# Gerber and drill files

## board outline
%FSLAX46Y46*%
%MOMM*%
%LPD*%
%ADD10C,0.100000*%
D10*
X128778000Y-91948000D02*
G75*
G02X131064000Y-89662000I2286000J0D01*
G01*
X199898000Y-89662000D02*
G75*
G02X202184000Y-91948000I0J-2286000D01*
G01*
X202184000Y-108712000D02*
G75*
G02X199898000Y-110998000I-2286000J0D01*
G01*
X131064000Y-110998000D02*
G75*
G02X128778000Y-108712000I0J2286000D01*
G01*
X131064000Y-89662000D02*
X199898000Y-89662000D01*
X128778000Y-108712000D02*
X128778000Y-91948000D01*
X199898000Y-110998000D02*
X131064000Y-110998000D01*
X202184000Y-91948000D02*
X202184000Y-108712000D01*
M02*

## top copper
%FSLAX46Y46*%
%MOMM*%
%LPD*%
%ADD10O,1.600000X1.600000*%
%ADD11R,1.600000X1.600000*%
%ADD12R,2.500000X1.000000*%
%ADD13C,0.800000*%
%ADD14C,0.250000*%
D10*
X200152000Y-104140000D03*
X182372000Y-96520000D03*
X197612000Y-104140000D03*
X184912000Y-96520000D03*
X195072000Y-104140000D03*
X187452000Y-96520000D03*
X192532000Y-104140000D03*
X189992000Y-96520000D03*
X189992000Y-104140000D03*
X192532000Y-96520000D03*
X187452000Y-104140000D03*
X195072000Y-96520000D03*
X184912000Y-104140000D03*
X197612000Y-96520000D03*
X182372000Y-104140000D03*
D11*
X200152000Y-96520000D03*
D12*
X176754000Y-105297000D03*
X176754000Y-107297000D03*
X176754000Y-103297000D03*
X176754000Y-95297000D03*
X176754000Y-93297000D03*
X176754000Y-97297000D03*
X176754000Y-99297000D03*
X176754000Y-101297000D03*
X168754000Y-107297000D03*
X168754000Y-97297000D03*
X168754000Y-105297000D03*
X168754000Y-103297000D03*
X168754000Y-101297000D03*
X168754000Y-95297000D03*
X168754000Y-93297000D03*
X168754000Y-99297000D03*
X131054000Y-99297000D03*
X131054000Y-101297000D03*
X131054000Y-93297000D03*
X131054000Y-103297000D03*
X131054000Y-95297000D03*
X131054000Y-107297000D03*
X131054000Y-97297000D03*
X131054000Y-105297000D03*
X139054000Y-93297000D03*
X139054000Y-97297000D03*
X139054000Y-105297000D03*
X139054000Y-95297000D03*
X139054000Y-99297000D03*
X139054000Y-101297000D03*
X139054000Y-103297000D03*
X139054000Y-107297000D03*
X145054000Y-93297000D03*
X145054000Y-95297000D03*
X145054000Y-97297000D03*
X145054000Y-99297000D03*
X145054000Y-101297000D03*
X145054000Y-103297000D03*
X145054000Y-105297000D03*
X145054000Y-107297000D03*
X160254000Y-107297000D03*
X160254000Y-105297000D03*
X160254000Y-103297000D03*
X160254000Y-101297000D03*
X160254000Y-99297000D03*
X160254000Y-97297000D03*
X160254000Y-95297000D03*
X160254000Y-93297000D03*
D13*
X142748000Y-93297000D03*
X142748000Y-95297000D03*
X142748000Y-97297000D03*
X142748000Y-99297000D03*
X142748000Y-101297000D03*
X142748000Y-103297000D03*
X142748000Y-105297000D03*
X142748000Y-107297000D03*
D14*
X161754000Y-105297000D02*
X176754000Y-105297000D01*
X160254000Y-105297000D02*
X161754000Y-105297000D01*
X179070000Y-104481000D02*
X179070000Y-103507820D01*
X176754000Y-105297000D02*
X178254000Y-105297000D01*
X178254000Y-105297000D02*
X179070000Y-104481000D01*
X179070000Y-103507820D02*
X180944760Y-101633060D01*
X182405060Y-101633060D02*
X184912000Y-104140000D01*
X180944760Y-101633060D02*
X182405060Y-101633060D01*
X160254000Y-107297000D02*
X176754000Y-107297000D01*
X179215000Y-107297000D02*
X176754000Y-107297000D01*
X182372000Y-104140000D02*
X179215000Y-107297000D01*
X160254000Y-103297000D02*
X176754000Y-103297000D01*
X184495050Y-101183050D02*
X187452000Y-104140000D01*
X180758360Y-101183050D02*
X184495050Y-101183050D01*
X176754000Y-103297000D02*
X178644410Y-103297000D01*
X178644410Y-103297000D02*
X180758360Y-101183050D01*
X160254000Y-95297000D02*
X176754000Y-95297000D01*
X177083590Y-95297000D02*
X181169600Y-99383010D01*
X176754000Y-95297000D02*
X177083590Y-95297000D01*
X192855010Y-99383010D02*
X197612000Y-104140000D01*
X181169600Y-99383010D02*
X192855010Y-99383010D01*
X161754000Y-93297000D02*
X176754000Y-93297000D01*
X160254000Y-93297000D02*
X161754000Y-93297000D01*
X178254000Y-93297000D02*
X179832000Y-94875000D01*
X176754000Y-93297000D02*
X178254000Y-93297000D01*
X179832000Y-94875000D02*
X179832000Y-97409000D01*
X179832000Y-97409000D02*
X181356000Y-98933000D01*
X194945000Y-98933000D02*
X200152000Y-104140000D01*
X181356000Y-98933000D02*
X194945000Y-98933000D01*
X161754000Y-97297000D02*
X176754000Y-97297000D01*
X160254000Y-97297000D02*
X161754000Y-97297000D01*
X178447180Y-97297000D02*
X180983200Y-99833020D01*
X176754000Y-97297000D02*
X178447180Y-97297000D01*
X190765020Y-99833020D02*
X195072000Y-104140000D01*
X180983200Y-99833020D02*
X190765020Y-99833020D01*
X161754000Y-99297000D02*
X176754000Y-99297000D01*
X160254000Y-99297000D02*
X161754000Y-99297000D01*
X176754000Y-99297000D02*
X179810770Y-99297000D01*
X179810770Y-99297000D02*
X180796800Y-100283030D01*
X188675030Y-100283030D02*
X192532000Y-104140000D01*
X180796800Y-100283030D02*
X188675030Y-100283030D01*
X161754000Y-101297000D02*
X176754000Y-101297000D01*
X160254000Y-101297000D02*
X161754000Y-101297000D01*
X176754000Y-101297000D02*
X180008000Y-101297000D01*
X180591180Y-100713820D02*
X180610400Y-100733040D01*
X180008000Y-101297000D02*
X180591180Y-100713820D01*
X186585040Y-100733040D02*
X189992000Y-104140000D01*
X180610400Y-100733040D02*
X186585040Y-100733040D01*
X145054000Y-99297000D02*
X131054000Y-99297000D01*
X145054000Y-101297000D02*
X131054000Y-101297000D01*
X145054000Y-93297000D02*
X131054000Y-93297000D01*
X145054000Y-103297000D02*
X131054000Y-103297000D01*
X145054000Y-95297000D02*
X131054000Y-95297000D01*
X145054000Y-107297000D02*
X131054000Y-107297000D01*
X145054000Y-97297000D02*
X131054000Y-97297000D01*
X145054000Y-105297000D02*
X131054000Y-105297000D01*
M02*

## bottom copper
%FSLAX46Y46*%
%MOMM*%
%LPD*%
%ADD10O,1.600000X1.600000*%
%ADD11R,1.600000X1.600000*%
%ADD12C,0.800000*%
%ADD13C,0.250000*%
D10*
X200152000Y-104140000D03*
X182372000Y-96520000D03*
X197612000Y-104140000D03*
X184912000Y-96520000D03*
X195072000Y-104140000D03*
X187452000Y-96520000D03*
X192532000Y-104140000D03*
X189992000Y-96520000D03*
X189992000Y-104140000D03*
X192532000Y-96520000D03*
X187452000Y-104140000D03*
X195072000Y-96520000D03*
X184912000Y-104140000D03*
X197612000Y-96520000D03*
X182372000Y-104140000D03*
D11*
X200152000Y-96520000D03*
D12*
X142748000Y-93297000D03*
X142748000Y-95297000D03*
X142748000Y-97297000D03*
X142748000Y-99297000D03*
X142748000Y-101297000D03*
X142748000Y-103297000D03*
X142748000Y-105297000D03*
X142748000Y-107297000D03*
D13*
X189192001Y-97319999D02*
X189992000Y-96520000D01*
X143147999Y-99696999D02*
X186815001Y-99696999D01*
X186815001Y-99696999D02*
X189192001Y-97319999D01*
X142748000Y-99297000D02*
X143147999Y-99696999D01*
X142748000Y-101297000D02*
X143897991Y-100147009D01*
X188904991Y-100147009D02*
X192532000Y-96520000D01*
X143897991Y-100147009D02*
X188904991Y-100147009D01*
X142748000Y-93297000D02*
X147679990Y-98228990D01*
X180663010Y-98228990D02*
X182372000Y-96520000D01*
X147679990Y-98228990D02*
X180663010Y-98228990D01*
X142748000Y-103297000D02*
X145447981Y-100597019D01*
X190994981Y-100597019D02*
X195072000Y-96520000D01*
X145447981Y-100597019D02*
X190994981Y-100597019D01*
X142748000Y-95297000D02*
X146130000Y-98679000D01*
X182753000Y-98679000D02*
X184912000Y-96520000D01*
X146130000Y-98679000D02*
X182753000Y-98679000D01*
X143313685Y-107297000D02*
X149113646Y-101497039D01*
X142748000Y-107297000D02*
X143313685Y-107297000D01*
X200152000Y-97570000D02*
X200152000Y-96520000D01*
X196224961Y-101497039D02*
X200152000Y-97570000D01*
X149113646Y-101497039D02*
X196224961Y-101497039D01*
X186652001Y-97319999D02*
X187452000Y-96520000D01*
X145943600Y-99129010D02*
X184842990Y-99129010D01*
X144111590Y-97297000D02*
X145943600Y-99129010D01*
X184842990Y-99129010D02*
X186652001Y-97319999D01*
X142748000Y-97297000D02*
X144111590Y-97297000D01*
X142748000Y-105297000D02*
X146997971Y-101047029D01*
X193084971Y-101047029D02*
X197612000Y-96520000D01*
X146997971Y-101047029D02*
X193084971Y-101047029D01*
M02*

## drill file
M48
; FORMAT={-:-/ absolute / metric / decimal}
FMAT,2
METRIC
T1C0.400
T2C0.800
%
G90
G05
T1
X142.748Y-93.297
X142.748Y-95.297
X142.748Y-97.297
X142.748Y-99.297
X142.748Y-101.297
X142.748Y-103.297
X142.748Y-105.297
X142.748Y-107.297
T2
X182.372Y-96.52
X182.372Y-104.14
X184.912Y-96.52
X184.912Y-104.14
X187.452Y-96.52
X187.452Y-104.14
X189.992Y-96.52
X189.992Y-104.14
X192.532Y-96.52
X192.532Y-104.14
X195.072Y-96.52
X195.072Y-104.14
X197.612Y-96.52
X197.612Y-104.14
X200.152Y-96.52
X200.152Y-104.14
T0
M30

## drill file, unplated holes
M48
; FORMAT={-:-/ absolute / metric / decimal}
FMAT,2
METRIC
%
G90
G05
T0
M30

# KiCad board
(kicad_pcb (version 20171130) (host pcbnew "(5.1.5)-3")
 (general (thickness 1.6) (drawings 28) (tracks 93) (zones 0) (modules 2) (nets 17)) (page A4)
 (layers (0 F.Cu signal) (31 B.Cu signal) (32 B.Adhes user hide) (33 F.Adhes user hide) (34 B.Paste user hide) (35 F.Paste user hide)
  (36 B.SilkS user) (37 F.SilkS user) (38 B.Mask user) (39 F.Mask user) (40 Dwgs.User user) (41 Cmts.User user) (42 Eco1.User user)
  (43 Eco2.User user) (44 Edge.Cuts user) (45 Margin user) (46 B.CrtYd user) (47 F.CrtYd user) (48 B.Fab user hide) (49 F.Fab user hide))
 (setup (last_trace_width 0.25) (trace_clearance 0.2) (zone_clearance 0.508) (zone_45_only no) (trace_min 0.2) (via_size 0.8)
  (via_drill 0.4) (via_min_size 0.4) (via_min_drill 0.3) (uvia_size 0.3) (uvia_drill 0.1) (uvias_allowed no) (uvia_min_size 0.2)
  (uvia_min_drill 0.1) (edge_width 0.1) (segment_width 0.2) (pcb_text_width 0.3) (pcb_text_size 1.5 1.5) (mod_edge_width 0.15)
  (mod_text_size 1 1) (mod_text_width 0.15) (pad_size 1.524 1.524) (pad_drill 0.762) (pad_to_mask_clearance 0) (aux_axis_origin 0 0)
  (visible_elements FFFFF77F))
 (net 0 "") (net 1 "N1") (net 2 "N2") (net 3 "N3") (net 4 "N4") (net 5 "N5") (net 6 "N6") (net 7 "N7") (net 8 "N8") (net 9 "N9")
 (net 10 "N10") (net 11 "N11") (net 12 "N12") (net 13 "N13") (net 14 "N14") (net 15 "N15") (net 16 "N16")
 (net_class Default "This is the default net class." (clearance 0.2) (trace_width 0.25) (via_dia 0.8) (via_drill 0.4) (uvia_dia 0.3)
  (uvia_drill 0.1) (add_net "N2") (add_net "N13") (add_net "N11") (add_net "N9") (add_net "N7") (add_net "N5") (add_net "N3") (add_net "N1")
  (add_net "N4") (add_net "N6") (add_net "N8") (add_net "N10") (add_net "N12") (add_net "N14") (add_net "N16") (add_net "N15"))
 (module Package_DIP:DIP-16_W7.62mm (layer F.Cu) (at 200.152 96.52 270)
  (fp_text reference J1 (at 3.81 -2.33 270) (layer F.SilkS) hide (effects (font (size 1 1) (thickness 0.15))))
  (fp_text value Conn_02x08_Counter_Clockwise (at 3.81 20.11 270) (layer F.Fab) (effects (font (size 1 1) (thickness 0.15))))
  (pad 16 thru_hole oval (at 7.62 0 270) (size 1.6 1.6) (drill 0.8) (layers *.Cu *.Mask) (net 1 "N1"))
  (pad 8 thru_hole oval (at 0 17.78 270) (size 1.6 1.6) (drill 0.8) (layers *.Cu *.Mask) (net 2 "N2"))
  (pad 15 thru_hole oval (at 7.62 2.54 270) (size 1.6 1.6) (drill 0.8) (layers *.Cu *.Mask) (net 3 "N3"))
  (pad 7 thru_hole oval (at 0 15.24 270) (size 1.6 1.6) (drill 0.8) (layers *.Cu *.Mask) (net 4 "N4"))
  (pad 14 thru_hole oval (at 7.62 5.08 270) (size 1.6 1.6) (drill 0.8) (layers *.Cu *.Mask) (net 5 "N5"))
  (pad 6 thru_hole oval (at 0 12.7 270) (size 1.6 1.6) (drill 0.8) (layers *.Cu *.Mask) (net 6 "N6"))
  (pad 13 thru_hole oval (at 7.62 7.62 270) (size 1.6 1.6) (drill 0.8) (layers *.Cu *.Mask) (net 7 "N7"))
  (pad 5 thru_hole oval (at 0 10.16 270) (size 1.6 1.6) (drill 0.8) (layers *.Cu *.Mask) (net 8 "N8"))
  (pad 12 thru_hole oval (at 7.62 10.16 270) (size 1.6 1.6) (drill 0.8) (layers *.Cu *.Mask) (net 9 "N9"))
  (pad 4 thru_hole oval (at 0 7.62 270) (size 1.6 1.6) (drill 0.8) (layers *.Cu *.Mask) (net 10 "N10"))
  (pad 11 thru_hole oval (at 7.62 12.7 270) (size 1.6 1.6) (drill 0.8) (layers *.Cu *.Mask) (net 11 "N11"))
  (pad 3 thru_hole oval (at 0 5.08 270) (size 1.6 1.6) (drill 0.8) (layers *.Cu *.Mask) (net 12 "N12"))
  (pad 10 thru_hole oval (at 7.62 15.24 270) (size 1.6 1.6) (drill 0.8) (layers *.Cu *.Mask) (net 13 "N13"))
  (pad 2 thru_hole oval (at 0 2.54 270) (size 1.6 1.6) (drill 0.8) (layers *.Cu *.Mask) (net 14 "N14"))
  (pad 9 thru_hole oval (at 7.62 17.78 270) (size 1.6 1.6) (drill 0.8) (layers *.Cu *.Mask) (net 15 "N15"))
  (pad 1 thru_hole rect (at 0 0 270) (size 1.6 1.6) (drill 0.8) (layers *.Cu *.Mask) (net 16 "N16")))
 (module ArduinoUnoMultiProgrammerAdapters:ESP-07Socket (layer F.Cu) (at 152.654 98.197)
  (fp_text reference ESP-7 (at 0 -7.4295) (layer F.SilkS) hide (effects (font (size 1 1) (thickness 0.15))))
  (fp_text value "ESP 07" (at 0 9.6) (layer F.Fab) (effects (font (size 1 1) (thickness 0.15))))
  (pad 10 smd rect (at 24.1 7.1) (size 2.5 1) (layers F.Cu F.Paste F.Mask) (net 13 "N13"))
  (pad 9 smd rect (at 24.1 9.1) (size 2.5 1) (layers F.Cu F.Paste F.Mask) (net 15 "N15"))
  (pad 11 smd rect (at 24.1 5.1) (size 2.5 1) (layers F.Cu F.Paste F.Mask) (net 11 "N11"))
  (pad 15 smd rect (at 24.1 -2.9) (size 2.5 1) (layers F.Cu F.Paste F.Mask) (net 3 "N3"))
  (pad 16 smd rect (at 24.1 -4.9) (size 2.5 1) (layers F.Cu F.Paste F.Mask) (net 1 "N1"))
  (pad 14 smd rect (at 24.1 -0.9) (size 2.5 1) (layers F.Cu F.Paste F.Mask) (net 5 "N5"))
  (pad 13 smd rect (at 24.1 1.1) (size 2.5 1) (layers F.Cu F.Paste F.Mask) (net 7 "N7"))
  (pad 12 smd rect (at 24.1 3.1) (size 2.5 1) (layers F.Cu F.Paste F.Mask) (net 9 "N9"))
  (pad 9 smd rect (at 16.1 9.1) (size 2.5 1) (layers F.Cu F.Paste F.Mask) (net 15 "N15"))
  (pad 14 smd rect (at 16.1 -0.9) (size 2.5 1) (layers F.Cu F.Paste F.Mask) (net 5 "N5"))
  (pad 10 smd rect (at 16.1 7.1) (size 2.5 1) (layers F.Cu F.Paste F.Mask) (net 13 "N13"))
  (pad 11 smd rect (at 16.1 5.1) (size 2.5 1) (layers F.Cu F.Paste F.Mask) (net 11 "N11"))
  (pad 12 smd rect (at 16.1 3.1) (size 2.5 1) (layers F.Cu F.Paste F.Mask) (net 9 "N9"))
  (pad 15 smd rect (at 16.1 -2.9) (size 2.5 1) (layers F.Cu F.Paste F.Mask) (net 3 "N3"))
  (pad 16 smd rect (at 16.1 -4.9) (size 2.5 1) (layers F.Cu F.Paste F.Mask) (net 1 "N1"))
  (pad 13 smd rect (at 16.1 1.1) (size 2.5 1) (layers F.Cu F.Paste F.Mask) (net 7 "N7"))
  (pad 4 smd rect (at -21.6 1.1) (size 2.5 1) (layers F.Cu F.Paste F.Mask) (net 8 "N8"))
  (pad 5 smd rect (at -21.6 3.1) (size 2.5 1) (layers F.Cu F.Paste F.Mask) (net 10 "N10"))
  (pad 1 smd rect (at -21.6 -4.9) (size 2.5 1) (layers F.Cu F.Paste F.Mask) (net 2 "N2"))
  (pad 6 smd rect (at -21.6 5.1) (size 2.5 1) (layers F.Cu F.Paste F.Mask) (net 12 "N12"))
  (pad 2 smd rect (at -21.6 -2.9) (size 2.5 1) (layers F.Cu F.Paste F.Mask) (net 4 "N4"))
  (pad 8 smd rect (at -21.6 9.1) (size 2.5 1) (layers F.Cu F.Paste F.Mask) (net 16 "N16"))
  (pad 3 smd rect (at -21.6 -0.9) (size 2.5 1) (layers F.Cu F.Paste F.Mask) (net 6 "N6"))
  (pad 7 smd rect (at -21.6 7.1) (size 2.5 1) (layers F.Cu F.Paste F.Mask) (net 14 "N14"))
  (pad 1 smd rect (at -13.6 -4.9) (size 2.5 1) (layers F.Cu F.Paste F.Mask) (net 2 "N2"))
  (pad 3 smd rect (at -13.6 -0.9) (size 2.5 1) (layers F.Cu F.Paste F.Mask) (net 6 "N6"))
  (pad 7 smd rect (at -13.6 7.1) (size 2.5 1) (layers F.Cu F.Paste F.Mask) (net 14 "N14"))
  (pad 2 smd rect (at -13.6 -2.9) (size 2.5 1) (layers F.Cu F.Paste F.Mask) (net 4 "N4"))
  (pad 4 smd rect (at -13.6 1.1) (size 2.5 1) (layers F.Cu F.Paste F.Mask) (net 8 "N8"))
  (pad 5 smd rect (at -13.6 3.1) (size 2.5 1) (layers F.Cu F.Paste F.Mask) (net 10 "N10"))
  (pad 6 smd rect (at -13.6 5.1) (size 2.5 1) (layers F.Cu F.Paste F.Mask) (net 12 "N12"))
  (pad 8 smd rect (at -13.6 9.1) (size 2.5 1) (layers F.Cu F.Paste F.Mask) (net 16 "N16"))
  (pad 1 smd rect (at -7.6 -4.9) (size 2.5 1) (layers F.Cu F.Paste F.Mask) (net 2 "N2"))
  (pad 2 smd rect (at -7.6 -2.9) (size 2.5 1) (layers F.Cu F.Paste F.Mask) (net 4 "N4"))
  (pad 3 smd rect (at -7.6 -0.9) (size 2.5 1) (layers F.Cu F.Paste F.Mask) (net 6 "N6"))
  (pad 4 smd rect (at -7.6 1.1) (size 2.5 1) (layers F.Cu F.Paste F.Mask) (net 8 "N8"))
  (pad 5 smd rect (at -7.6 3.1) (size 2.5 1) (layers F.Cu F.Paste F.Mask) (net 10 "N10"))
  (pad 6 smd rect (at -7.6 5.1) (size 2.5 1) (layers F.Cu F.Paste F.Mask) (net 12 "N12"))
  (pad 7 smd rect (at -7.6 7.1) (size 2.5 1) (layers F.Cu F.Paste F.Mask) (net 14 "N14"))
  (pad 8 smd rect (at -7.6 9.1) (size 2.5 1) (layers F.Cu F.Paste F.Mask) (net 16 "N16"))
  (pad 9 smd rect (at 7.6 9.1) (size 2.5 1) (layers F.Cu F.Paste F.Mask) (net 15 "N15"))
  (pad 10 smd rect (at 7.6 7.1) (size 2.5 1) (layers F.Cu F.Paste F.Mask) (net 13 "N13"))
  (pad 11 smd rect (at 7.6 5.1) (size 2.5 1) (layers F.Cu F.Paste F.Mask) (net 11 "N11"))
  (pad 12 smd rect (at 7.6 3.1) (size 2.5 1) (layers F.Cu F.Paste F.Mask) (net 9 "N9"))
  (pad 13 smd rect (at 7.6 1.1) (size 2.5 1) (layers F.Cu F.Paste F.Mask) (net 7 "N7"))
  (pad 14 smd rect (at 7.6 -0.9) (size 2.5 1) (layers F.Cu F.Paste F.Mask) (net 5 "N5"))
  (pad 15 smd rect (at 7.6 -2.9) (size 2.5 1) (layers F.Cu F.Paste F.Mask) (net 3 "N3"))
  (pad 16 smd rect (at 7.6 -4.9) (size 2.5 1) (layers F.Cu F.Paste F.Mask) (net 1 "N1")))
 (gr_arc (start 131.064 91.948) (end 131.064 89.662) (angle -90) (layer Edge.Cuts) (width 0.1))
 (gr_arc (start 199.898 91.948) (end 202.184 91.948) (angle -90) (layer Edge.Cuts) (width 0.1))
 (gr_arc (start 199.898 108.712) (end 199.898 110.998) (angle -90) (layer Edge.Cuts) (width 0.1))
 (gr_arc (start 131.064 108.712) (end 128.778 108.712) (angle -90) (layer Edge.Cuts) (width 0.1))
 (gr_line (start 131.064 89.662) (end 199.898 89.662) (layer Edge.Cuts) (width 0.1))
 (gr_line (start 128.778 108.712) (end 128.778 91.948) (layer Edge.Cuts) (width 0.1))
 (gr_line (start 199.898 110.998) (end 131.064 110.998) (layer Edge.Cuts) (width 0.1))
 (gr_line (start 202.184 91.948) (end 202.184 108.712) (layer Edge.Cuts) (width 0.1))
 (via (at 142.748 93.297) (size 0.8) (drill 0.4) (layers F.Cu B.Cu) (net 2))
 (via (at 142.748 95.297) (size 0.8) (drill 0.4) (layers F.Cu B.Cu) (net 4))
 (via (at 142.748 97.297) (size 0.8) (drill 0.4) (layers F.Cu B.Cu) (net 6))
 (via (at 142.748 99.297) (size 0.8) (drill 0.4) (layers F.Cu B.Cu) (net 8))
 (via (at 142.748 101.297) (size 0.8) (drill 0.4) (layers F.Cu B.Cu) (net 10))
 (via (at 142.748 103.297) (size 0.8) (drill 0.4) (layers F.Cu B.Cu) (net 12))
 (via (at 142.748 105.297) (size 0.8) (drill 0.4) (layers F.Cu B.Cu) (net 14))
 (via (at 142.748 107.297) (size 0.8) (drill 0.4) (layers F.Cu B.Cu) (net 16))
 (segment (start 161.754 105.297) (end 176.754 105.297) (width 0.25) (layer F.Cu) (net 13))
 (segment (start 160.254 105.297) (end 161.754 105.297) (width 0.25) (layer F.Cu) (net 13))
 (segment (start 179.07 104.481) (end 179.07 103.50782) (width 0.25) (layer F.Cu) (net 13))
 (segment (start 176.754 105.297) (end 178.254 105.297) (width 0.25) (layer F.Cu) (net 13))
 (segment (start 178.254 105.297) (end 179.07 104.481) (width 0.25) (layer F.Cu) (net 13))
 (segment (start 179.07 103.50782) (end 180.94476 101.63306) (width 0.25) (layer F.Cu) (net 13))
 (segment (start 182.40506 101.63306) (end 184.912 104.14) (width 0.25) (layer F.Cu) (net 13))
 (segment (start 180.94476 101.63306) (end 182.40506 101.63306) (width 0.25) (layer F.Cu) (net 13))
 (segment (start 160.254 107.297) (end 176.754 107.297) (width 0.25) (layer F.Cu) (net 15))
 (segment (start 179.215 107.297) (end 176.754 107.297) (width 0.25) (layer F.Cu) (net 15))
 (segment (start 182.372 104.14) (end 179.215 107.297) (width 0.25) (layer F.Cu) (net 15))
 (segment (start 160.254 103.297) (end 176.754 103.297) (width 0.25) (layer F.Cu) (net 11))
 (segment (start 184.49505 101.18305) (end 187.452 104.14) (width 0.25) (layer F.Cu) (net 11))
 (segment (start 180.75836 101.18305) (end 184.49505 101.18305) (width 0.25) (layer F.Cu) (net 11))
 (segment (start 176.754 103.297) (end 178.64441 103.297) (width 0.25) (layer F.Cu) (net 11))
 (segment (start 178.64441 103.297) (end 180.75836 101.18305) (width 0.25) (layer F.Cu) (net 11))
 (segment (start 160.254 95.297) (end 176.754 95.297) (width 0.25) (layer F.Cu) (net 3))
 (segment (start 177.08359 95.297) (end 181.1696 99.38301) (width 0.25) (layer F.Cu) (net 3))
 (segment (start 176.754 95.297) (end 177.08359 95.297) (width 0.25) (layer F.Cu) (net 3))
 (segment (start 192.85501 99.38301) (end 197.612 104.14) (width 0.25) (layer F.Cu) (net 3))
 (segment (start 181.1696 99.38301) (end 192.85501 99.38301) (width 0.25) (layer F.Cu) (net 3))
 (segment (start 161.754 93.297) (end 176.754 93.297) (width 0.25) (layer F.Cu) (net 1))
 (segment (start 160.254 93.297) (end 161.754 93.297) (width 0.25) (layer F.Cu) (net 1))
 (segment (start 178.254 93.297) (end 179.832 94.875) (width 0.25) (layer F.Cu) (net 1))
 (segment (start 176.754 93.297) (end 178.254 93.297) (width 0.25) (layer F.Cu) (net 1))
 (segment (start 179.832 94.875) (end 179.832 97.409) (width 0.25) (layer F.Cu) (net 1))
 (segment (start 179.832 97.409) (end 181.356 98.933) (width 0.25) (layer F.Cu) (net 1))
 (segment (start 194.945 98.933) (end 200.152 104.14) (width 0.25) (layer F.Cu) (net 1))
 (segment (start 181.356 98.933) (end 194.945 98.933) (width 0.25) (layer F.Cu) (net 1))
 (segment (start 161.754 97.297) (end 176.754 97.297) (width 0.25) (layer F.Cu) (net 5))
 (segment (start 160.254 97.297) (end 161.754 97.297) (width 0.25) (layer F.Cu) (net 5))
 (segment (start 178.44718 97.297) (end 180.9832 99.83302) (width 0.25) (layer F.Cu) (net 5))
 (segment (start 176.754 97.297) (end 178.44718 97.297) (width 0.25) (layer F.Cu) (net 5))
 (segment (start 190.76502 99.83302) (end 195.072 104.14) (width 0.25) (layer F.Cu) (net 5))
 (segment (start 180.9832 99.83302) (end 190.76502 99.83302) (width 0.25) (layer F.Cu) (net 5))
 (segment (start 161.754 99.297) (end 176.754 99.297) (width 0.25) (layer F.Cu) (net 7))
 (segment (start 160.254 99.297) (end 161.754 99.297) (width 0.25) (layer F.Cu) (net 7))
 (segment (start 176.754 99.297) (end 179.81077 99.297) (width 0.25) (layer F.Cu) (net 7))
 (segment (start 179.81077 99.297) (end 180.7968 100.28303) (width 0.25) (layer F.Cu) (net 7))
 (segment (start 188.67503 100.28303) (end 192.532 104.14) (width 0.25) (layer F.Cu) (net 7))
 (segment (start 180.7968 100.28303) (end 188.67503 100.28303) (width 0.25) (layer F.Cu) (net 7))
 (segment (start 161.754 101.297) (end 176.754 101.297) (width 0.25) (layer F.Cu) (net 9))
 (segment (start 160.254 101.297) (end 161.754 101.297) (width 0.25) (layer F.Cu) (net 9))
 (segment (start 176.754 101.297) (end 180.008 101.297) (width 0.25) (layer F.Cu) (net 9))
 (segment (start 180.59118 100.71382) (end 180.6104 100.73304) (width 0.25) (layer F.Cu) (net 9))
 (segment (start 180.008 101.297) (end 180.59118 100.71382) (width 0.25) (layer F.Cu) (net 9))
 (segment (start 186.58504 100.73304) (end 189.992 104.14) (width 0.25) (layer F.Cu) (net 9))
 (segment (start 180.6104 100.73304) (end 186.58504 100.73304) (width 0.25) (layer F.Cu) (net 9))
 (segment (start 145.054 99.297) (end 131.054 99.297) (width 0.25) (layer F.Cu) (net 8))
 (segment (start 189.192001 97.319999) (end 189.992 96.52) (width 0.25) (layer B.Cu) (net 8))
 (segment (start 143.147999 99.696999) (end 186.815001 99.696999) (width 0.25) (layer B.Cu) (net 8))
 (segment (start 186.815001 99.696999) (end 189.192001 97.319999) (width 0.25) (layer B.Cu) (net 8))
 (segment (start 142.748 99.297) (end 143.147999 99.696999) (width 0.25) (layer B.Cu) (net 8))
 (segment (start 145.054 101.297) (end 131.054 101.297) (width 0.25) (layer F.Cu) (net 10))
 (segment (start 142.748 101.297) (end 143.897991 100.147009) (width 0.25) (layer B.Cu) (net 10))
 (segment (start 188.904991 100.147009) (end 192.532 96.52) (width 0.25) (layer B.Cu) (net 10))
 (segment (start 143.897991 100.147009) (end 188.904991 100.147009) (width 0.25) (layer B.Cu) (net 10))
 (segment (start 145.054 93.297) (end 131.054 93.297) (width 0.25) (layer F.Cu) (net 2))
 (segment (start 142.748 93.297) (end 147.67999 98.22899) (width 0.25) (layer B.Cu) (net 2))
 (segment (start 180.66301 98.22899) (end 182.372 96.52) (width 0.25) (layer B.Cu) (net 2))
 (segment (start 147.67999 98.22899) (end 180.66301 98.22899) (width 0.25) (layer B.Cu) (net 2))
 (segment (start 145.054 103.297) (end 131.054 103.297) (width 0.25) (layer F.Cu) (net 12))
 (segment (start 142.748 103.297) (end 145.447981 100.597019) (width 0.25) (layer B.Cu) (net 12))
 (segment (start 190.994981 100.597019) (end 195.072 96.52) (width 0.25) (layer B.Cu) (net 12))
 (segment (start 145.447981 100.597019) (end 190.994981 100.597019) (width 0.25) (layer B.Cu) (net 12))
 (segment (start 145.054 95.297) (end 131.054 95.297) (width 0.25) (layer F.Cu) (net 4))
 (segment (start 142.748 95.297) (end 146.13 98.679) (width 0.25) (layer B.Cu) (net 4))
 (segment (start 182.753 98.679) (end 184.912 96.52) (width 0.25) (layer B.Cu) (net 4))
 (segment (start 146.13 98.679) (end 182.753 98.679) (width 0.25) (layer B.Cu) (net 4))
 (segment (start 145.054 107.297) (end 131.054 107.297) (width 0.25) (layer F.Cu) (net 16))
 (segment (start 143.313685 107.297) (end 149.113646 101.497039) (width 0.25) (layer B.Cu) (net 16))
 (segment (start 142.748 107.297) (end 143.313685 107.297) (width 0.25) (layer B.Cu) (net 16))
 (segment (start 200.152 97.57) (end 200.152 96.52) (width 0.25) (layer B.Cu) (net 16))
 (segment (start 196.224961 101.497039) (end 200.152 97.57) (width 0.25) (layer B.Cu) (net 16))
 (segment (start 149.113646 101.497039) (end 196.224961 101.497039) (width 0.25) (layer B.Cu) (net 16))
 (segment (start 145.054 97.297) (end 131.054 97.297) (width 0.25) (layer F.Cu) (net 6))
 (segment (start 186.652001 97.319999) (end 187.452 96.52) (width 0.25) (layer B.Cu) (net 6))
 (segment (start 145.9436 99.12901) (end 184.84299 99.12901) (width 0.25) (layer B.Cu) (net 6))
 (segment (start 144.11159 97.297) (end 145.9436 99.12901) (width 0.25) (layer B.Cu) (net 6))
 (segment (start 184.84299 99.12901) (end 186.652001 97.319999) (width 0.25) (layer B.Cu) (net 6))
 (segment (start 142.748 97.297) (end 144.11159 97.297) (width 0.25) (layer B.Cu) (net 6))
 (segment (start 145.054 105.297) (end 131.054 105.297) (width 0.25) (layer F.Cu) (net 14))
 (segment (start 142.748 105.297) (end 146.997971 101.047029) (width 0.25) (layer B.Cu) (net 14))
 (segment (start 193.084971 101.047029) (end 197.612 96.52) (width 0.25) (layer B.Cu) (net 14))
 (segment (start 146.997971 101.047029) (end 193.084971 101.047029) (width 0.25) (layer B.Cu) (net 14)))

